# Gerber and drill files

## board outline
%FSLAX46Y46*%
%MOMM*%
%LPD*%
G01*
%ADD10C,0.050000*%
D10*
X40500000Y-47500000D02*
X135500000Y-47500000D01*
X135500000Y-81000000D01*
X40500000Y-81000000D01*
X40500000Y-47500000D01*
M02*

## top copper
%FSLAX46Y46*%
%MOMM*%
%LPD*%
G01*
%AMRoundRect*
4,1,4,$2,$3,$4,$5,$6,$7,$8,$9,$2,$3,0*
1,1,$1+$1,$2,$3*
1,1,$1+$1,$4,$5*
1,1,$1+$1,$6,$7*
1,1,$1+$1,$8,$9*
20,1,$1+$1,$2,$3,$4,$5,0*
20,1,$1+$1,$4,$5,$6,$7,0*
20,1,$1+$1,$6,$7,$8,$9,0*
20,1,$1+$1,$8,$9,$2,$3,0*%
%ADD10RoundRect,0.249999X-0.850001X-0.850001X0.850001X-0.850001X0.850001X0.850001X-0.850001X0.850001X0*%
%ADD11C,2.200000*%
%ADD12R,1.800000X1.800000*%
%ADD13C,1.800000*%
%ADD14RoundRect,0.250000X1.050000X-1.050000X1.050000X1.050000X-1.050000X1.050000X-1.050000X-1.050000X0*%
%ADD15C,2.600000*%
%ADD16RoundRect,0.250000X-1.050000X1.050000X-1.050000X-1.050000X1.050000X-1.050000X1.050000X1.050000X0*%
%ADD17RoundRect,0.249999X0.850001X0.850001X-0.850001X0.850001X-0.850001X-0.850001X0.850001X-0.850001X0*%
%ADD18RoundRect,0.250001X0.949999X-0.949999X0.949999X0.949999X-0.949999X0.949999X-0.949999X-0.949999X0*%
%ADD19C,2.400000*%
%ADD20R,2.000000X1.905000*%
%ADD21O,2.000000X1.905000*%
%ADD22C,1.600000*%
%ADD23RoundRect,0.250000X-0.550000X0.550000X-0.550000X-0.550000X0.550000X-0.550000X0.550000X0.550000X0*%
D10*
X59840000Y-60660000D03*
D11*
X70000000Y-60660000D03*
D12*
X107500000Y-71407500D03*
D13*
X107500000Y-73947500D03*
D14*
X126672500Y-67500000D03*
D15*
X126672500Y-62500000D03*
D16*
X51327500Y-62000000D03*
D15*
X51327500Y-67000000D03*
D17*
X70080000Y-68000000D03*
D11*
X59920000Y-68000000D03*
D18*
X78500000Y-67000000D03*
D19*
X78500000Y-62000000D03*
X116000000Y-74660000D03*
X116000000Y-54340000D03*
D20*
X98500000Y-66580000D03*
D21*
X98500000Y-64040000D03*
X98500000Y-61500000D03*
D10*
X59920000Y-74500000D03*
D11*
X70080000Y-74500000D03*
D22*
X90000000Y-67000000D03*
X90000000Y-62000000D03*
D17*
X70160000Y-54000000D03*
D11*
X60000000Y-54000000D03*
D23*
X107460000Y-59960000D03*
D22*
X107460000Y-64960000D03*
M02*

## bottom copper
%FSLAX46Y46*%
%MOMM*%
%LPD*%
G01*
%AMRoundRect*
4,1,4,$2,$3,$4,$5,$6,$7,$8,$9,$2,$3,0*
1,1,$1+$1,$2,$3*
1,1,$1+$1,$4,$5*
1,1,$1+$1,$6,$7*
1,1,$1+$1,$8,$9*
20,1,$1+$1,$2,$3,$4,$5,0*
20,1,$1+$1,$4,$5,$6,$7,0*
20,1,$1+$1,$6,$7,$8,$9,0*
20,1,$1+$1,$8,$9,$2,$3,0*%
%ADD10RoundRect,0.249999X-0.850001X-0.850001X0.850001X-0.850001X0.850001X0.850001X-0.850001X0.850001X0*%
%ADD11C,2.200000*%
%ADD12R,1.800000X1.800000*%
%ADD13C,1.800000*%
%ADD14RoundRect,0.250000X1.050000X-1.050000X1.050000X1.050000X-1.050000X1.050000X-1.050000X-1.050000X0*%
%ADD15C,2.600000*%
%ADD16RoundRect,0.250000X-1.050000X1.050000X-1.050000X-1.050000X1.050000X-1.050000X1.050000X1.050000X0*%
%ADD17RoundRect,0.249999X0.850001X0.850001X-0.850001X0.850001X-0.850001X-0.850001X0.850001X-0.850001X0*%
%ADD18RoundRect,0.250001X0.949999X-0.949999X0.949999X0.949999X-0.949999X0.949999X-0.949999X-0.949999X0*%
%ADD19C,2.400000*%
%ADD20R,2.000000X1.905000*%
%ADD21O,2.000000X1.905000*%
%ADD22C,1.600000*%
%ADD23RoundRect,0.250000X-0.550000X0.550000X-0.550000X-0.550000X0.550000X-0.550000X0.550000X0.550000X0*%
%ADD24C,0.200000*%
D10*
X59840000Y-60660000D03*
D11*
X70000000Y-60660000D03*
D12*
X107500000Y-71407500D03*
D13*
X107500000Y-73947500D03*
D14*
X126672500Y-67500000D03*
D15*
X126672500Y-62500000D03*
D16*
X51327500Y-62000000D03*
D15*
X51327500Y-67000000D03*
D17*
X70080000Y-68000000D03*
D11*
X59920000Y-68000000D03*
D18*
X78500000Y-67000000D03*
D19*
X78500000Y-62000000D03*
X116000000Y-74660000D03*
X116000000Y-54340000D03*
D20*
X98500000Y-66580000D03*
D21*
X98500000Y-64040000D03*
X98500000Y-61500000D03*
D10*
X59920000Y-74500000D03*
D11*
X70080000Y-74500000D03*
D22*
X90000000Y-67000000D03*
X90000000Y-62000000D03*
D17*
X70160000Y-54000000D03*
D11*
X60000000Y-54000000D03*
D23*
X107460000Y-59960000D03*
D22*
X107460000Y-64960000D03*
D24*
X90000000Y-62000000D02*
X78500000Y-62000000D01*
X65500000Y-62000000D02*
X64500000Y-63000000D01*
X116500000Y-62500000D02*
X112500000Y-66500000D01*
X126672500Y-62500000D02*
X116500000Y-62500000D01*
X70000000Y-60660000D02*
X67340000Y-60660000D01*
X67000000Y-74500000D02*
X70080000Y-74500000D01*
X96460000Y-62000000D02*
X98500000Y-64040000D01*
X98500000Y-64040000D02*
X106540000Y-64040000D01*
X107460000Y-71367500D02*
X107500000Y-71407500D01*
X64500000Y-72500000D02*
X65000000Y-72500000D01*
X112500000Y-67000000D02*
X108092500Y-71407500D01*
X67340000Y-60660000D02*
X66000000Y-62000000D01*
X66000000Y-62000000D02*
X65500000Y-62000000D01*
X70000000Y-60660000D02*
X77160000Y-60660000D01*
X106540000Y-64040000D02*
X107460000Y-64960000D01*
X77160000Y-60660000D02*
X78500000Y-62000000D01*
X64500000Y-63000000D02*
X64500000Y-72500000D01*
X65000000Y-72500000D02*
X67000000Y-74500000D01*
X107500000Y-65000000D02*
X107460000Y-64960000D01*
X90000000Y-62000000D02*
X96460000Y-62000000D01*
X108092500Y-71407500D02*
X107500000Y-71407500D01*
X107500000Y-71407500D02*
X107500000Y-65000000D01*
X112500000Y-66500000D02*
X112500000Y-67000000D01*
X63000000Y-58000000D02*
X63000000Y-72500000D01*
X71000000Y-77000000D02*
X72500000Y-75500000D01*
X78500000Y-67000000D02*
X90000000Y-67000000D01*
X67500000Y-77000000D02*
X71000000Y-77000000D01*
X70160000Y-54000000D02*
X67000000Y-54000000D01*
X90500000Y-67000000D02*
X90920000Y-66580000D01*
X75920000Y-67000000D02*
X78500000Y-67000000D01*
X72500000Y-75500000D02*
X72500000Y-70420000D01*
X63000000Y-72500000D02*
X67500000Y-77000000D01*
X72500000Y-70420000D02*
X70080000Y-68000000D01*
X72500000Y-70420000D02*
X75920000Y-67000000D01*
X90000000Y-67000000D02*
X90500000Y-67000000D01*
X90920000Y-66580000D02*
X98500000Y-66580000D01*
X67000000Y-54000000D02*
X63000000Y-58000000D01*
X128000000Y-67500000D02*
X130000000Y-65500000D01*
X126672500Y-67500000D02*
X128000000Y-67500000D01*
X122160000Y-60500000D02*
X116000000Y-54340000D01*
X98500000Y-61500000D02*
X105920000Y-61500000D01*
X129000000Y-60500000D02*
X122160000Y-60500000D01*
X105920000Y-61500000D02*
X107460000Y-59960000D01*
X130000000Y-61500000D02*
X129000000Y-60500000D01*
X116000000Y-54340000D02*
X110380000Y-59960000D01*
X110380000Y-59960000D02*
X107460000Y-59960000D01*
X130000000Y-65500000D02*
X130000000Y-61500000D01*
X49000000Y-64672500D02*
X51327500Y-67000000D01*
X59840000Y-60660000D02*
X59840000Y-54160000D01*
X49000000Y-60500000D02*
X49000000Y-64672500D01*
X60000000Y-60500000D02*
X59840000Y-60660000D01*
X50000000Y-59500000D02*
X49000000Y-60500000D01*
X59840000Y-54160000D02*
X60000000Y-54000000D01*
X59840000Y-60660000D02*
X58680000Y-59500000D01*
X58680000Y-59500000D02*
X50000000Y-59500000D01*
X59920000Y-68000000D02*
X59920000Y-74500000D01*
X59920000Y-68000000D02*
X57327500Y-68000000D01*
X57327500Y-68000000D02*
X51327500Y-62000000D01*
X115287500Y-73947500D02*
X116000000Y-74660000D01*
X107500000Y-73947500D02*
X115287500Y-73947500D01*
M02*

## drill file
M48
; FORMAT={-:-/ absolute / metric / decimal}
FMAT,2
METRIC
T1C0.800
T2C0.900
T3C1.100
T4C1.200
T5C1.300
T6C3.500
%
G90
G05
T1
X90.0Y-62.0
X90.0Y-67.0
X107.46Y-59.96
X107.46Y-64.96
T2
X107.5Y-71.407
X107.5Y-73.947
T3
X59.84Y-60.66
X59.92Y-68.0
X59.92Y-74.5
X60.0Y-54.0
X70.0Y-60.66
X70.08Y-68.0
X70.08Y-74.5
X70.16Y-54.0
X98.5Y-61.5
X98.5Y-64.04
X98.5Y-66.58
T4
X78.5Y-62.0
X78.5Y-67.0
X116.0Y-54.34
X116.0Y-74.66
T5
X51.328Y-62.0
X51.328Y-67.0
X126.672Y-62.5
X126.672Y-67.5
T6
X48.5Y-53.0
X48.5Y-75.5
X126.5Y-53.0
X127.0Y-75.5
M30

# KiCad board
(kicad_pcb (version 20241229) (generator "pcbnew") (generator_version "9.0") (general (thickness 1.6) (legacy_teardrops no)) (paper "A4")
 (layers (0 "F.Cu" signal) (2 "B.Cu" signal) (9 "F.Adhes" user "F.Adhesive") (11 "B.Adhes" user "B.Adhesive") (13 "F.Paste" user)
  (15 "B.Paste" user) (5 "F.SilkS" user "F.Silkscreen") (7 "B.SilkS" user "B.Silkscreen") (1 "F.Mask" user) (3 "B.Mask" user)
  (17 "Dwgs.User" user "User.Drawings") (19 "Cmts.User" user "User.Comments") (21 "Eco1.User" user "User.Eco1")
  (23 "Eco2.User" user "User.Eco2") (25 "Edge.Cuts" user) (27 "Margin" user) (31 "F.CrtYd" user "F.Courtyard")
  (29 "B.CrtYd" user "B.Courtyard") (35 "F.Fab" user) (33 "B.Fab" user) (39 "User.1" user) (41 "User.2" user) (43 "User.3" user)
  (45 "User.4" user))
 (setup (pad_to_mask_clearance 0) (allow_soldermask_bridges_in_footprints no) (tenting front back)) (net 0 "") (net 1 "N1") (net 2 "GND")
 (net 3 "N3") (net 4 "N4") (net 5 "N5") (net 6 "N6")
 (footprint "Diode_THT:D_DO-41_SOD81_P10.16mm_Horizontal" (layer "F.Cu") (at 59.84 60.66)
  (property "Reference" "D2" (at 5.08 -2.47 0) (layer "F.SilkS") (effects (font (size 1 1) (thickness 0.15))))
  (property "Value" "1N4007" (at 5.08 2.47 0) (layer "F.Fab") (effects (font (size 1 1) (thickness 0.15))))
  (pad "1" thru_hole roundrect (at 0 0) (size 2.2 2.2) (drill 1.1) (layers "*.Cu" "*.Mask") (remove_unused_layers no)
   (roundrect_rratio 0.113636) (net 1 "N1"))
  (pad "2" thru_hole circle (at 10.16 0) (size 2.2 2.2) (drill 1.1) (layers "*.Cu" "*.Mask") (remove_unused_layers no) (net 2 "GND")))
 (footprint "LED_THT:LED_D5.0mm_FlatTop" (layer "F.Cu") (at 107.5 71.4075 -90)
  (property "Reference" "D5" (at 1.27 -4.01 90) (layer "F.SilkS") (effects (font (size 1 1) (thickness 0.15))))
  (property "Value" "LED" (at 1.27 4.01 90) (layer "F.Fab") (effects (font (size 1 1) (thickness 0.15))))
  (pad "1" thru_hole rect (at 0 0 270) (size 1.8 1.8) (drill 0.9) (layers "*.Cu" "*.Mask") (remove_unused_layers no) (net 2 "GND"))
  (pad "2" thru_hole circle (at 2.54 0 270) (size 1.8 1.8) (drill 0.9) (layers "*.Cu" "*.Mask") (remove_unused_layers no) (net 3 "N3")))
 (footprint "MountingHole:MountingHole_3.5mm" (layer "F.Cu") (at 127 75.5)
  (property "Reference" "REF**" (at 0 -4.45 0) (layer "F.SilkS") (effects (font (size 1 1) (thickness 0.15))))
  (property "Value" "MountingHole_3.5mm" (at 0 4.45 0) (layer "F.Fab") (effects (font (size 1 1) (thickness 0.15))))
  (pad "" np_thru_hole circle (at 0 0) (size 3.5 3.5) (drill 3.5) (layers "*.Cu" "*.Mask")))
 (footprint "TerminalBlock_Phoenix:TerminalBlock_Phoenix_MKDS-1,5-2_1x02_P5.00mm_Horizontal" (layer "F.Cu") (at 126.6725 67.5 90)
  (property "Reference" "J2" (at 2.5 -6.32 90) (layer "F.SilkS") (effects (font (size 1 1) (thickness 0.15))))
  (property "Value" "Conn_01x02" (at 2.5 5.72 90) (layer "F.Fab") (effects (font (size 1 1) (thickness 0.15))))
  (pad "1" thru_hole roundrect (at 0 0 90) (size 2.6 2.6) (drill 1.3) (layers "*.Cu" "*.Mask") (remove_unused_layers no)
   (roundrect_rratio 0.096154) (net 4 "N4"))
  (pad "2" thru_hole circle (at 5 0 90) (size 2.6 2.6) (drill 1.3) (layers "*.Cu" "*.Mask") (remove_unused_layers no) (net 2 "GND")))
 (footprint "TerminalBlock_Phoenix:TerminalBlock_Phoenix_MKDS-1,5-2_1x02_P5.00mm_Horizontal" (layer "F.Cu") (at 51.3275 62 -90)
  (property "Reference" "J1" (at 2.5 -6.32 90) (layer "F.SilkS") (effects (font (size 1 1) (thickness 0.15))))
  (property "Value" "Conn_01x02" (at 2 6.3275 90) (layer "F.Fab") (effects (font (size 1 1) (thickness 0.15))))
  (pad "1" thru_hole roundrect (at 0 0 270) (size 2.6 2.6) (drill 1.3) (layers "*.Cu" "*.Mask") (remove_unused_layers no)
   (roundrect_rratio 0.096154) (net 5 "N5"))
  (pad "2" thru_hole circle (at 5 0 270) (size 2.6 2.6) (drill 1.3) (layers "*.Cu" "*.Mask") (remove_unused_layers no) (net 1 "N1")))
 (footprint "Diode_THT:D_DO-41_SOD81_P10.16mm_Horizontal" (layer "F.Cu") (at 70.08 68 180)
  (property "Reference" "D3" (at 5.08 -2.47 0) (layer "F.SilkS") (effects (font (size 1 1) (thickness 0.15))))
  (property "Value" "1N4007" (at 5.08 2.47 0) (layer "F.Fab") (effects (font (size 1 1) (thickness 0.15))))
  (pad "1" thru_hole roundrect (at 0 0 180) (size 2.2 2.2) (drill 1.1) (layers "*.Cu" "*.Mask") (remove_unused_layers no)
   (roundrect_rratio 0.113636) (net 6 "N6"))
  (pad "2" thru_hole circle (at 10.16 0 180) (size 2.2 2.2) (drill 1.1) (layers "*.Cu" "*.Mask") (remove_unused_layers no) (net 5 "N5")))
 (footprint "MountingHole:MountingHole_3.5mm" (layer "F.Cu") (at 48.5 75.5)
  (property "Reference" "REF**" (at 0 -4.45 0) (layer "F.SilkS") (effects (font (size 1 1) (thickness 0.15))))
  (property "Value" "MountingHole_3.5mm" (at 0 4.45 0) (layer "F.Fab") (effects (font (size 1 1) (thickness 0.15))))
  (pad "" np_thru_hole circle (at 0 0) (size 3.5 3.5) (drill 3.5) (layers "*.Cu" "*.Mask")))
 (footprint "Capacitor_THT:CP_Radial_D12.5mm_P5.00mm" (layer "F.Cu") (at 78.5 67 90)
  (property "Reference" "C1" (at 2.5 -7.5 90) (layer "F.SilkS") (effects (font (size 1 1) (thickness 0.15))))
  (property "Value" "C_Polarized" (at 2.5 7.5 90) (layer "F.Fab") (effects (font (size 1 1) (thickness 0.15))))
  (pad "1" thru_hole roundrect (at 0 0 90) (size 2.4 2.4) (drill 1.2) (layers "*.Cu" "*.Mask") (remove_unused_layers no)
   (roundrect_rratio 0.104167) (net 6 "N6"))
  (pad "2" thru_hole circle (at 5 0 90) (size 2.4 2.4) (drill 1.2) (layers "*.Cu" "*.Mask") (remove_unused_layers no) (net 2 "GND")))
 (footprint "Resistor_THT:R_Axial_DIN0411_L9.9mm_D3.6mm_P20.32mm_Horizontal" (layer "F.Cu") (at 116 74.66 90)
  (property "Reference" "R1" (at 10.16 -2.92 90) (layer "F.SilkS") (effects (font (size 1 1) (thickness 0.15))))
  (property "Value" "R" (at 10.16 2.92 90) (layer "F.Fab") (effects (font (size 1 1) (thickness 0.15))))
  (pad "1" thru_hole circle (at 0 0 90) (size 2.4 2.4) (drill 1.2) (layers "*.Cu" "*.Mask") (remove_unused_layers no) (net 3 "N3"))
  (pad "2" thru_hole circle (at 20.32 0 90) (size 2.4 2.4) (drill 1.2) (layers "*.Cu" "*.Mask") (remove_unused_layers no) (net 4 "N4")))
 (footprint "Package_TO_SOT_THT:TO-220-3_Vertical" (layer "F.Cu") (at 98.5 66.58 90)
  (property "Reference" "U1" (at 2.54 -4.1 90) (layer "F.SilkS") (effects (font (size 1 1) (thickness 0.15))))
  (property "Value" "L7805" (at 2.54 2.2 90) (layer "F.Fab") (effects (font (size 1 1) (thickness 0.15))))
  (pad "1" thru_hole rect (at 0 0 90) (size 1.905 2) (drill 1.1) (layers "*.Cu" "*.Mask") (remove_unused_layers no) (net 6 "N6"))
  (pad "2" thru_hole oval (at 2.54 0 90) (size 1.905 2) (drill 1.1) (layers "*.Cu" "*.Mask") (remove_unused_layers no) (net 2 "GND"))
  (pad "3" thru_hole oval (at 5.08 0 90) (size 1.905 2) (drill 1.1) (layers "*.Cu" "*.Mask") (remove_unused_layers no) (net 4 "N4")))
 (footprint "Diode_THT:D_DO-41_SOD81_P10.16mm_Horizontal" (layer "F.Cu") (at 59.92 74.5)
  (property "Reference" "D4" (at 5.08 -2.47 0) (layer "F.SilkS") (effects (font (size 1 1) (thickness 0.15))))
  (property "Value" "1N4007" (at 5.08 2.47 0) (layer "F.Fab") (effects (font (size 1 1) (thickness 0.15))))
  (pad "1" thru_hole roundrect (at 0 0) (size 2.2 2.2) (drill 1.1) (layers "*.Cu" "*.Mask") (remove_unused_layers no)
   (roundrect_rratio 0.113636) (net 5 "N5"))
  (pad "2" thru_hole circle (at 10.16 0) (size 2.2 2.2) (drill 1.1) (layers "*.Cu" "*.Mask") (remove_unused_layers no) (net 2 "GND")))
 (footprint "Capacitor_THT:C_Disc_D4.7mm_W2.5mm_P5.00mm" (layer "F.Cu") (at 90 67 90)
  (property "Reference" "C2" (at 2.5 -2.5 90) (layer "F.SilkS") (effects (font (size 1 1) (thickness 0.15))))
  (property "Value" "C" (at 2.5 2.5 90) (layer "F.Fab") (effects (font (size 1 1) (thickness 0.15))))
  (pad "1" thru_hole circle (at 0 0 90) (size 1.6 1.6) (drill 0.8) (layers "*.Cu" "*.Mask") (remove_unused_layers no) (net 6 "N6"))
  (pad "2" thru_hole circle (at 5 0 90) (size 1.6 1.6) (drill 0.8) (layers "*.Cu" "*.Mask") (remove_unused_layers no) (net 2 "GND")))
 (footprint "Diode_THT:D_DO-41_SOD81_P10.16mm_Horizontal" (layer "F.Cu") (at 70.16 54 180)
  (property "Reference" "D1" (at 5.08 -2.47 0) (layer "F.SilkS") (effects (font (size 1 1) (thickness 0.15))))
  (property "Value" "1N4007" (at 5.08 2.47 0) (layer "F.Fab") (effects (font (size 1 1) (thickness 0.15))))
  (pad "1" thru_hole roundrect (at 0 0 180) (size 2.2 2.2) (drill 1.1) (layers "*.Cu" "*.Mask") (remove_unused_layers no)
   (roundrect_rratio 0.113636) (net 6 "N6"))
  (pad "2" thru_hole circle (at 10.16 0 180) (size 2.2 2.2) (drill 1.1) (layers "*.Cu" "*.Mask") (remove_unused_layers no) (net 1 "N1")))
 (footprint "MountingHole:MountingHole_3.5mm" (layer "F.Cu") (at 48.5 53)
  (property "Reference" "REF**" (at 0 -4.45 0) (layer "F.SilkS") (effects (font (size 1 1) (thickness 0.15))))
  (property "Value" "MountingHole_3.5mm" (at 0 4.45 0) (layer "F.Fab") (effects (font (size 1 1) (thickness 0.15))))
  (pad "" np_thru_hole circle (at 0 0) (size 3.5 3.5) (drill 3.5) (layers "*.Cu" "*.Mask")))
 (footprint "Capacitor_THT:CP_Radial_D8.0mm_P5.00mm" (layer "F.Cu") (at 107.46 59.96 -90)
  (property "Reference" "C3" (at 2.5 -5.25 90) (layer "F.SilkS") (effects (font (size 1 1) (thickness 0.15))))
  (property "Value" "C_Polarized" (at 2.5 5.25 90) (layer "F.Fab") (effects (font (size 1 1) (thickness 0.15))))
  (pad "1" thru_hole roundrect (at 0 0 270) (size 1.6 1.6) (drill 0.8) (layers "*.Cu" "*.Mask") (remove_unused_layers no)
   (roundrect_rratio 0.15625) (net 4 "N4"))
  (pad "2" thru_hole circle (at 5 0 270) (size 1.6 1.6) (drill 0.8) (layers "*.Cu" "*.Mask") (remove_unused_layers no) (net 2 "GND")))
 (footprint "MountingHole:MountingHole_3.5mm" (layer "F.Cu") (at 126.5 53)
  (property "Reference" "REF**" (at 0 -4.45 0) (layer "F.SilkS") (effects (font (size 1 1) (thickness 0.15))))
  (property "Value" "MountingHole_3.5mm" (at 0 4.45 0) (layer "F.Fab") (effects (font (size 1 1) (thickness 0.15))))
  (pad "" np_thru_hole circle (at 0 0) (size 3.5 3.5) (drill 3.5) (layers "*.Cu" "*.Mask")))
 (gr_rect (start 40.5 47.5) (end 135.5 81) (stroke (width 0.05) (type default)) (fill no) (layer "Edge.Cuts"))
 (segment (start 90 62) (end 78.5 62) (width 0.2) (layer "B.Cu") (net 2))
 (segment (start 65.5 62) (end 64.5 63) (width 0.2) (layer "B.Cu") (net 2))
 (segment (start 116.5 62.5) (end 112.5 66.5) (width 0.2) (layer "B.Cu") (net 2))
 (segment (start 126.6725 62.5) (end 116.5 62.5) (width 0.2) (layer "B.Cu") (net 2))
 (segment (start 70 60.66) (end 67.34 60.66) (width 0.2) (layer "B.Cu") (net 2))
 (segment (start 67 74.5) (end 70.08 74.5) (width 0.2) (layer "B.Cu") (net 2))
 (segment (start 96.46 62) (end 98.5 64.04) (width 0.2) (layer "B.Cu") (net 2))
 (segment (start 98.5 64.04) (end 106.54 64.04) (width 0.2) (layer "B.Cu") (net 2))
 (segment (start 107.46 71.3675) (end 107.5 71.4075) (width 0.2) (layer "B.Cu") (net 2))
 (segment (start 64.5 72.5) (end 65 72.5) (width 0.2) (layer "B.Cu") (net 2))
 (segment (start 112.5 67) (end 108.0925 71.4075) (width 0.2) (layer "B.Cu") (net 2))
 (segment (start 67.34 60.66) (end 66 62) (width 0.2) (layer "B.Cu") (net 2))
 (segment (start 66 62) (end 65.5 62) (width 0.2) (layer "B.Cu") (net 2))
 (segment (start 70 60.66) (end 77.16 60.66) (width 0.2) (layer "B.Cu") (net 2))
 (segment (start 106.54 64.04) (end 107.46 64.96) (width 0.2) (layer "B.Cu") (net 2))
 (segment (start 77.16 60.66) (end 78.5 62) (width 0.2) (layer "B.Cu") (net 2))
 (segment (start 64.5 63) (end 64.5 72.5) (width 0.2) (layer "B.Cu") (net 2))
 (segment (start 65 72.5) (end 67 74.5) (width 0.2) (layer "B.Cu") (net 2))
 (segment (start 107.5 65) (end 107.46 64.96) (width 0.2) (layer "B.Cu") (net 2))
 (segment (start 90 62) (end 96.46 62) (width 0.2) (layer "B.Cu") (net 2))
 (segment (start 108.0925 71.4075) (end 107.5 71.4075) (width 0.2) (layer "B.Cu") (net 2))
 (segment (start 107.5 71.4075) (end 107.5 65) (width 0.2) (layer "B.Cu") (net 2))
 (segment (start 112.5 66.5) (end 112.5 67) (width 0.2) (layer "B.Cu") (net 2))
 (segment (start 63 58) (end 63 72.5) (width 0.2) (layer "B.Cu") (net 6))
 (segment (start 71 77) (end 72.5 75.5) (width 0.2) (layer "B.Cu") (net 6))
 (segment (start 78.5 67) (end 90 67) (width 0.2) (layer "B.Cu") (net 6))
 (segment (start 67.5 77) (end 71 77) (width 0.2) (layer "B.Cu") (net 6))
 (segment (start 70.16 54) (end 67 54) (width 0.2) (layer "B.Cu") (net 6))
 (segment (start 90.5 67) (end 90.92 66.58) (width 0.2) (layer "B.Cu") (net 6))
 (segment (start 75.92 67) (end 78.5 67) (width 0.2) (layer "B.Cu") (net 6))
 (segment (start 72.5 75.5) (end 72.5 70.42) (width 0.2) (layer "B.Cu") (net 6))
 (segment (start 63 72.5) (end 67.5 77) (width 0.2) (layer "B.Cu") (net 6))
 (segment (start 72.5 70.42) (end 70.08 68) (width 0.2) (layer "B.Cu") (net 6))
 (segment (start 72.5 70.42) (end 75.92 67) (width 0.2) (layer "B.Cu") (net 6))
 (segment (start 90 67) (end 90.5 67) (width 0.2) (layer "B.Cu") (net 6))
 (segment (start 90.92 66.58) (end 98.5 66.58) (width 0.2) (layer "B.Cu") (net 6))
 (segment (start 67 54) (end 63 58) (width 0.2) (layer "B.Cu") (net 6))
 (segment (start 128 67.5) (end 130 65.5) (width 0.2) (layer "B.Cu") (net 4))
 (segment (start 126.6725 67.5) (end 128 67.5) (width 0.2) (layer "B.Cu") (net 4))
 (segment (start 122.16 60.5) (end 116 54.34) (width 0.2) (layer "B.Cu") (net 4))
 (segment (start 98.5 61.5) (end 105.92 61.5) (width 0.2) (layer "B.Cu") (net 4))
 (segment (start 129 60.5) (end 122.16 60.5) (width 0.2) (layer "B.Cu") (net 4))
 (segment (start 105.92 61.5) (end 107.46 59.96) (width 0.2) (layer "B.Cu") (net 4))
 (segment (start 130 61.5) (end 129 60.5) (width 0.2) (layer "B.Cu") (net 4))
 (segment (start 116 54.34) (end 110.38 59.96) (width 0.2) (layer "B.Cu") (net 4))
 (segment (start 110.38 59.96) (end 107.46 59.96) (width 0.2) (layer "B.Cu") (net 4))
 (segment (start 130 65.5) (end 130 61.5) (width 0.2) (layer "B.Cu") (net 4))
 (segment (start 49 64.6725) (end 51.3275 67) (width 0.2) (layer "B.Cu") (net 1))
 (segment (start 59.84 60.66) (end 59.84 54.16) (width 0.2) (layer "B.Cu") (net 1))
 (segment (start 49 60.5) (end 49 64.6725) (width 0.2) (layer "B.Cu") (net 1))
 (segment (start 60 60.5) (end 59.84 60.66) (width 0.2) (layer "B.Cu") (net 1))
 (segment (start 50 59.5) (end 49 60.5) (width 0.2) (layer "B.Cu") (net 1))
 (segment (start 59.84 54.16) (end 60 54) (width 0.2) (layer "B.Cu") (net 1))
 (segment (start 59.84 60.66) (end 58.68 59.5) (width 0.2) (layer "B.Cu") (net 1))
 (segment (start 58.68 59.5) (end 50 59.5) (width 0.2) (layer "B.Cu") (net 1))
 (segment (start 59.92 68) (end 59.92 74.5) (width 0.2) (layer "B.Cu") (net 5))
 (segment (start 59.92 68) (end 57.3275 68) (width 0.2) (layer "B.Cu") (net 5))
 (segment (start 57.3275 68) (end 51.3275 62) (width 0.2) (layer "B.Cu") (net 5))
 (segment (start 115.2875 73.9475) (end 116 74.66) (width 0.2) (layer "B.Cu") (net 3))
 (segment (start 107.5 73.9475) (end 115.2875 73.9475) (width 0.2) (layer "B.Cu") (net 3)))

